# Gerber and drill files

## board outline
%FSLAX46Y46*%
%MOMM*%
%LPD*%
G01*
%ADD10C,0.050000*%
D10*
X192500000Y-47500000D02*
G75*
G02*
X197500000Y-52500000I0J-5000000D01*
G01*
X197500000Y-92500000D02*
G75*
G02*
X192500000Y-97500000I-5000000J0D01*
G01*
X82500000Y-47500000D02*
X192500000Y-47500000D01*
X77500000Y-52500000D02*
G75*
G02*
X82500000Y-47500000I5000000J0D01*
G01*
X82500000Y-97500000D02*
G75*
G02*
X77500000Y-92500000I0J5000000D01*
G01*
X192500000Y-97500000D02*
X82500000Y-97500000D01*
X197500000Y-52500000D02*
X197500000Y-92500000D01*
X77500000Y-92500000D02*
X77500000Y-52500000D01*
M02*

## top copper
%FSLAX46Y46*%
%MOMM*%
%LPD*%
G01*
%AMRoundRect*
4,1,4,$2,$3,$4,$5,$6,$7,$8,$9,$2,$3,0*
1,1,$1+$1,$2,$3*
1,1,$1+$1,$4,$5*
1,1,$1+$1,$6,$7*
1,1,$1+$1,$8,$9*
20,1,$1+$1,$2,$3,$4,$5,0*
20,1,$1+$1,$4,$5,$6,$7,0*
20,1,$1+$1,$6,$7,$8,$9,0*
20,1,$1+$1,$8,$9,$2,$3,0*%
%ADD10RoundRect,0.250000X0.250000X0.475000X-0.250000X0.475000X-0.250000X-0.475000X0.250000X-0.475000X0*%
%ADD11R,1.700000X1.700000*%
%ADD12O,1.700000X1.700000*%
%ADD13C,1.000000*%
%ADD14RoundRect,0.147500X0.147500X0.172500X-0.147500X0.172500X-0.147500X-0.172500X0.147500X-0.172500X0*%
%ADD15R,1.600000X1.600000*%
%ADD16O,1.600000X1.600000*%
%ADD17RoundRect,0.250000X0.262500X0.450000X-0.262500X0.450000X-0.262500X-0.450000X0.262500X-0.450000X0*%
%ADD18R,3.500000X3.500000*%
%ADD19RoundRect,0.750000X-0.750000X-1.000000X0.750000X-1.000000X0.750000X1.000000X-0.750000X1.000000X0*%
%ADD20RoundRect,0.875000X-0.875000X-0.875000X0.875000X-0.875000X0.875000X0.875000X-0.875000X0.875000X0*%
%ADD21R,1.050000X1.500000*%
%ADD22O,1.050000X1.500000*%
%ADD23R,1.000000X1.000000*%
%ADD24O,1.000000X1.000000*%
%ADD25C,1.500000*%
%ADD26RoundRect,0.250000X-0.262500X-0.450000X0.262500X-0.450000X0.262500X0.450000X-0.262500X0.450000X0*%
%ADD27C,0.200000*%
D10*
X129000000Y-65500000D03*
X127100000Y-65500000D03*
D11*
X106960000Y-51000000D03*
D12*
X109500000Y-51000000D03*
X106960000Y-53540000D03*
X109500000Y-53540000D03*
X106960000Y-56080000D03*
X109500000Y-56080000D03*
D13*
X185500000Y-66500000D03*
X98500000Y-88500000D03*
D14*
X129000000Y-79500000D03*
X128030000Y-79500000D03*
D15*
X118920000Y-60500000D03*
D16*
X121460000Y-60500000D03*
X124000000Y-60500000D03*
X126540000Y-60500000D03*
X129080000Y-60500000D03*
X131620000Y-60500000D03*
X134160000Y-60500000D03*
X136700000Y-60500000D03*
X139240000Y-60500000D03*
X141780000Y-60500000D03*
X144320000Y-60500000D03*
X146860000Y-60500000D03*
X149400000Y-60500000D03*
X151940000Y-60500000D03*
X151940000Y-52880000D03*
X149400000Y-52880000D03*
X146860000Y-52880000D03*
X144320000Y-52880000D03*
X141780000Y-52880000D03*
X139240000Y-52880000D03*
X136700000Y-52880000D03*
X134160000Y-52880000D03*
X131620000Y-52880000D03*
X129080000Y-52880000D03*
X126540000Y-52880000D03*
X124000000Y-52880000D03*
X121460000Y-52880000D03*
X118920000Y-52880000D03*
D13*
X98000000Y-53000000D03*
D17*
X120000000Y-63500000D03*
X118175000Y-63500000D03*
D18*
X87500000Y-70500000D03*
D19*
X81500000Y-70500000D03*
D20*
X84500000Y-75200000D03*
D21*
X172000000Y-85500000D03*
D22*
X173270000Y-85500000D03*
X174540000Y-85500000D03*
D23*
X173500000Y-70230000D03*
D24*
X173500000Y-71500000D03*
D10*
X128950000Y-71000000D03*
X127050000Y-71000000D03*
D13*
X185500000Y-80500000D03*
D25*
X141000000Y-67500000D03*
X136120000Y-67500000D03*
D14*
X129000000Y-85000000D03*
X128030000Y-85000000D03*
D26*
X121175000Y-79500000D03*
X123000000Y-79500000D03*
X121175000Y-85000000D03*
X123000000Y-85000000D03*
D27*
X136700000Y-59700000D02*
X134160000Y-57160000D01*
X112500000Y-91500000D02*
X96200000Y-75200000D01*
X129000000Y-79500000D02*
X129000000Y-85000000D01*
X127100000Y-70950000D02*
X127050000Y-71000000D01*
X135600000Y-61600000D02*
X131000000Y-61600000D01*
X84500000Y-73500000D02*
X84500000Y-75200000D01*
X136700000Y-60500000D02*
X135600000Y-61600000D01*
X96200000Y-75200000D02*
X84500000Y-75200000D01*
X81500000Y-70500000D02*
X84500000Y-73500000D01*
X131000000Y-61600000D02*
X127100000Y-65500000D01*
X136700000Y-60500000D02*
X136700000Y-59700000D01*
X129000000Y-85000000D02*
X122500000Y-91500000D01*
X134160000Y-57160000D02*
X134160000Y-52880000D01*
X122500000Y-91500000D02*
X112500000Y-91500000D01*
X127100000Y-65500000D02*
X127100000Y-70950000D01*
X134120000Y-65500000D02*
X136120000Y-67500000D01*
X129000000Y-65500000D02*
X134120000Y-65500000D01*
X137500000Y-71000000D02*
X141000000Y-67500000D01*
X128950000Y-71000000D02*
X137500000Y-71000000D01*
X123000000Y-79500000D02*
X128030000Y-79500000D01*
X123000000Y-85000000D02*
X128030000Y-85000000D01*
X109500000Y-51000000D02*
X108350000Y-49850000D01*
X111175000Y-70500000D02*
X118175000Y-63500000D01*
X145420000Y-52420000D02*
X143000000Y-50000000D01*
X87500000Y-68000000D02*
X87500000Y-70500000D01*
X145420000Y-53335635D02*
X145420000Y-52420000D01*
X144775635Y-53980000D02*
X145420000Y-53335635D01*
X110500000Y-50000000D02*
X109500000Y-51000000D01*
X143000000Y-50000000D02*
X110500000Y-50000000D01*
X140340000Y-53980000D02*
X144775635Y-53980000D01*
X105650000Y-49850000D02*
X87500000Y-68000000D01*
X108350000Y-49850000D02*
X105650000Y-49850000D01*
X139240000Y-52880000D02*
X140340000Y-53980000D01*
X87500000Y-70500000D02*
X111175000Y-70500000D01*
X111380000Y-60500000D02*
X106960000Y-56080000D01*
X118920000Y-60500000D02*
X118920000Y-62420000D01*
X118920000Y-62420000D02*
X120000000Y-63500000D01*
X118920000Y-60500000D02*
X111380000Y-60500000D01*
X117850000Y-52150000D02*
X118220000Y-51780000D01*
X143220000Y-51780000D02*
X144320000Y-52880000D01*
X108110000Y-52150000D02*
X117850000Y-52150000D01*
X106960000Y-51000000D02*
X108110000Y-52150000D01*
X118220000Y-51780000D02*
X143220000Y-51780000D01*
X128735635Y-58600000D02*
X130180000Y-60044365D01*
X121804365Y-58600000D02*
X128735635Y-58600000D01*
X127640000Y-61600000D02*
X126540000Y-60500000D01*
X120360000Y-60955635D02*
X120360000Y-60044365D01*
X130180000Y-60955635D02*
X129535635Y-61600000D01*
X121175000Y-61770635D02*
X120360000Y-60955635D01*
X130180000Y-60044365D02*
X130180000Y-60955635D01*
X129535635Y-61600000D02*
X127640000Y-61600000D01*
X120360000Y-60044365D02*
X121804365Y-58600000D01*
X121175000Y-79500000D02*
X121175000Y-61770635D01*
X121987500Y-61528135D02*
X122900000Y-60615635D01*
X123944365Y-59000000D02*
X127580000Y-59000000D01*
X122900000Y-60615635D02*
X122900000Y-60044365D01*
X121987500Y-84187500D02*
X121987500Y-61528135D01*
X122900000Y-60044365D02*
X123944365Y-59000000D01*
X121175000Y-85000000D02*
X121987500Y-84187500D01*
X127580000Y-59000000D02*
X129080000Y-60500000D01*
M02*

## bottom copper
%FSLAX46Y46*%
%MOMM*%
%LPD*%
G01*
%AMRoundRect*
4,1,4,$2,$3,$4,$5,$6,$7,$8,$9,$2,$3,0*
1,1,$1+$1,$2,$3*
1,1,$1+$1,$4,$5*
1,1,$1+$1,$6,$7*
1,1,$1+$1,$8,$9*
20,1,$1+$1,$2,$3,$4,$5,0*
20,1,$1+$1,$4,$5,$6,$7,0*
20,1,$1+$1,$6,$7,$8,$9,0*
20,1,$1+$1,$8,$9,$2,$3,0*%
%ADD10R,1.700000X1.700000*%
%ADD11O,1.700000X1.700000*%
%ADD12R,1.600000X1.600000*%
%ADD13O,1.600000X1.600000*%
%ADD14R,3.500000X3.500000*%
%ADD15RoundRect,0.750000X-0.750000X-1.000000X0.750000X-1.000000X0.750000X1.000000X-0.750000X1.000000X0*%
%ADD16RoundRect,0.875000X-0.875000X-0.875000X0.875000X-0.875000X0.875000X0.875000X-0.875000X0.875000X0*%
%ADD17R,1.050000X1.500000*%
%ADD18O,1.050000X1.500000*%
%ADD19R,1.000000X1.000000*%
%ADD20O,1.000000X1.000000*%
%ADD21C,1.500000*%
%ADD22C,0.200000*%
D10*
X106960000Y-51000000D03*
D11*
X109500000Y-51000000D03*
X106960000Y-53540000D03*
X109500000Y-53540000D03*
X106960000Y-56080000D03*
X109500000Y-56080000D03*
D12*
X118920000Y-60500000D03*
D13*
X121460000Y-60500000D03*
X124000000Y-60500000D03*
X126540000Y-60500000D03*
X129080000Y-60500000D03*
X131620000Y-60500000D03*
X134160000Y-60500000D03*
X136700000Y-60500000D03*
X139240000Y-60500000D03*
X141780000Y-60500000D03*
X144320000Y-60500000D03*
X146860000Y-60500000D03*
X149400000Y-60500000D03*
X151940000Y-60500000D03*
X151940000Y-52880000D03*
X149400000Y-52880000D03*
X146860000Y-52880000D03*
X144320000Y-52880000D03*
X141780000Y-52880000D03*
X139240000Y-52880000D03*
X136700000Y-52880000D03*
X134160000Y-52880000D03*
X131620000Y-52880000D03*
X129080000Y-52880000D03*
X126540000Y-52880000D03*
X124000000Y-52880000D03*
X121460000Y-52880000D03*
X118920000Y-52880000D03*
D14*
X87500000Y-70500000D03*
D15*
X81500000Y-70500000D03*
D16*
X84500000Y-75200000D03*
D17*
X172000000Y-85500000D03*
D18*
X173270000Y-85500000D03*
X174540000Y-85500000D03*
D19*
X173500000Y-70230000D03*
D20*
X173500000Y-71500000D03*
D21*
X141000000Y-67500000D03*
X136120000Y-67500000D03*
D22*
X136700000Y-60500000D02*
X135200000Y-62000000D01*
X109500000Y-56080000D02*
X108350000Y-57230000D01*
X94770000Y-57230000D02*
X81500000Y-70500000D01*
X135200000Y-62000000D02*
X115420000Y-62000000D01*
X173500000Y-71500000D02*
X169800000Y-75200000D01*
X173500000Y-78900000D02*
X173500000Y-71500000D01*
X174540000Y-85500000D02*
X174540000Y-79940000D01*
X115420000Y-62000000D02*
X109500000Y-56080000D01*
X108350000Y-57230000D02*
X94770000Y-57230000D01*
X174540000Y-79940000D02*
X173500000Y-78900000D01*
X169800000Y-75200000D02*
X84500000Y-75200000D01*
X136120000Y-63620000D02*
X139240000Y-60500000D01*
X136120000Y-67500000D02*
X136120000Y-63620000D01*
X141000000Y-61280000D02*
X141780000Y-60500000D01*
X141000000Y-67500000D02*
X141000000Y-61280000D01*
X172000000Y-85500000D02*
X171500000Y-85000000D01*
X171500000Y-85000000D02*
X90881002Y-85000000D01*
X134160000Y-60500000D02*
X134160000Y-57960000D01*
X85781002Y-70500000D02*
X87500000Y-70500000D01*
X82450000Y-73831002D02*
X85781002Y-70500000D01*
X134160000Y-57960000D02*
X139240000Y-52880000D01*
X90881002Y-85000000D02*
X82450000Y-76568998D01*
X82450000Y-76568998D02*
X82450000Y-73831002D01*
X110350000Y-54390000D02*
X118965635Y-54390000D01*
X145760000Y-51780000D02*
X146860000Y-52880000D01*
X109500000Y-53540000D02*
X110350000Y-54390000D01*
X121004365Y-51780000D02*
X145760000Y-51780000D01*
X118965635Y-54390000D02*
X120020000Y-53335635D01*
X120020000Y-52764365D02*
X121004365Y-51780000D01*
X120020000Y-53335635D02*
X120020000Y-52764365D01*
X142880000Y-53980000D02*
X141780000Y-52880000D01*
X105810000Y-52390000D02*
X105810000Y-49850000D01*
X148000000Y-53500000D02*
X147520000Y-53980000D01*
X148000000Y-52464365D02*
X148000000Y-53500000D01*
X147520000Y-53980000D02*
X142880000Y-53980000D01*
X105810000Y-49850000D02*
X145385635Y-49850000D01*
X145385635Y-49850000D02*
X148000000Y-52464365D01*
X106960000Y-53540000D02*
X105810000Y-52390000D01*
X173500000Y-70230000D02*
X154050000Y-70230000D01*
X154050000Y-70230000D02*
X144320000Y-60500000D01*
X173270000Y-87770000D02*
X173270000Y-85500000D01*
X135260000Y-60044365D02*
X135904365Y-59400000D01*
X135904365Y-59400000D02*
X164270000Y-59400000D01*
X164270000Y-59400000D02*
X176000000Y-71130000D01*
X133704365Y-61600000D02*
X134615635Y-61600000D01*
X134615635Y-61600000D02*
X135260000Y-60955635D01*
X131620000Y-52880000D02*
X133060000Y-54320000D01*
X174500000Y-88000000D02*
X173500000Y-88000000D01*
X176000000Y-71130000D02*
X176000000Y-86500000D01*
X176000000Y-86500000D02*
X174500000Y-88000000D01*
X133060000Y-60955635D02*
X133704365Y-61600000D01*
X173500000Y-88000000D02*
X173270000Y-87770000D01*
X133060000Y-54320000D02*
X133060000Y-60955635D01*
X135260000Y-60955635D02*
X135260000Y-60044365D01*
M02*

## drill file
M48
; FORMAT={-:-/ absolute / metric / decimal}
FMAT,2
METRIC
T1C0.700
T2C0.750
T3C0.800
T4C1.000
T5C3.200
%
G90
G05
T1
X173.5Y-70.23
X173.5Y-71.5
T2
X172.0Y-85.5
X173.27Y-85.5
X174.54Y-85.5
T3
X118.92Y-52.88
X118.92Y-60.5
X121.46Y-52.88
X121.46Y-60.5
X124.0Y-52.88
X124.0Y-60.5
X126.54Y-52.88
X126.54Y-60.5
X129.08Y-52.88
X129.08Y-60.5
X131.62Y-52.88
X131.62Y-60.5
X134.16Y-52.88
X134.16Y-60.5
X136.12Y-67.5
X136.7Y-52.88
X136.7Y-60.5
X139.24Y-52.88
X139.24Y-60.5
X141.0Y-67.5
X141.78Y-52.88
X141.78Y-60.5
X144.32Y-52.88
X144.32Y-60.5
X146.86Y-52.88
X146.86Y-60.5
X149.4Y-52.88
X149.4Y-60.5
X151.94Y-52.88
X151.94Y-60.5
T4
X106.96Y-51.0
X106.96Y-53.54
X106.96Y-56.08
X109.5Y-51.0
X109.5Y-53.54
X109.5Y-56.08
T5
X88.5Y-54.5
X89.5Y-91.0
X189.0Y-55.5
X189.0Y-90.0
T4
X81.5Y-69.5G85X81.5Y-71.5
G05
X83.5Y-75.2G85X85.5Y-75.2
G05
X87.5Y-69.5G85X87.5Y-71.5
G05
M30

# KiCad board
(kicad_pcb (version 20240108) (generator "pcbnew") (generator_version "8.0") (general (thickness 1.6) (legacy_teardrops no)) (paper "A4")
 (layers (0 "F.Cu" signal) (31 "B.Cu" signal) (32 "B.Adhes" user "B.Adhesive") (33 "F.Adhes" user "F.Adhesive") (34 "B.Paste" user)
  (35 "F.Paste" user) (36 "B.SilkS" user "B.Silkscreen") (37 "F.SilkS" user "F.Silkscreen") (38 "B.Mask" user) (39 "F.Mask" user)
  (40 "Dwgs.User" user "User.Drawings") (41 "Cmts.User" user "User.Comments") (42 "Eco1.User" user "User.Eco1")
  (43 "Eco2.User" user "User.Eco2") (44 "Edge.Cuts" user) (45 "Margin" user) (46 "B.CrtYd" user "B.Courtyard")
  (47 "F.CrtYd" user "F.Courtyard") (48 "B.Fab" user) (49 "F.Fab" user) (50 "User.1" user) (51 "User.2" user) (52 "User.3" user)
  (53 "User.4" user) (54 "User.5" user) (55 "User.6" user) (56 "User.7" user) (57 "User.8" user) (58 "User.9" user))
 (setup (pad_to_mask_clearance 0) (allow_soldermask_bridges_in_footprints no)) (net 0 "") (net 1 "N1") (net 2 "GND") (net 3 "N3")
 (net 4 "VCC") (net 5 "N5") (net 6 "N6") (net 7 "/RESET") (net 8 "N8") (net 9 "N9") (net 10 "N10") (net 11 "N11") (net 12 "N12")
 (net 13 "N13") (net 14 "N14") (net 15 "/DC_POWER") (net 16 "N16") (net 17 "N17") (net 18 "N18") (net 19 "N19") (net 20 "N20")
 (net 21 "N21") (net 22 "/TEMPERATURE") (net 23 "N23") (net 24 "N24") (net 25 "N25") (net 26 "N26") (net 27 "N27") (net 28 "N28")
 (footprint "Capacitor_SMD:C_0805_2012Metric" (layer "F.Cu") (at 128.05 65.5 180)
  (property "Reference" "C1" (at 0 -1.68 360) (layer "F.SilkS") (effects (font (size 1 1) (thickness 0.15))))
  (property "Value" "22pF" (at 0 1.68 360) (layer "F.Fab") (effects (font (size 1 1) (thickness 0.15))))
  (pad "1" smd roundrect (at -0.95 0 180) (size 1 1.45) (layers "F.Cu" "F.Paste" "F.Mask") (roundrect_rratio 0.25) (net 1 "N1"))
  (pad "2" smd roundrect (at 0.95 0 180) (size 1 1.45) (layers "F.Cu" "F.Paste" "F.Mask") (roundrect_rratio 0.25) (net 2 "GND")))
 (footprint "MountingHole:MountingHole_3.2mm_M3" (layer "F.Cu") (at 189 55.5)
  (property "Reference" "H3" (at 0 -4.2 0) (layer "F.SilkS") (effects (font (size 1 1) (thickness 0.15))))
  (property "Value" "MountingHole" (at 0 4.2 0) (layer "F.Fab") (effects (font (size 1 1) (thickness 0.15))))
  (pad "" np_thru_hole circle (at 0 0) (size 3.2 3.2) (drill 3.2) (layers "*.Cu" "*.Mask")))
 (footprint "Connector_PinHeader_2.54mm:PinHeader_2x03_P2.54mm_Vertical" (layer "F.Cu") (at 106.96 51)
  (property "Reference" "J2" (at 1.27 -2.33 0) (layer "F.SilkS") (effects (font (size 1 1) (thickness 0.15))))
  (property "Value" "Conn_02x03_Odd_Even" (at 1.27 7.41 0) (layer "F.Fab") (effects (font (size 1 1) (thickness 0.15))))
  (pad "1" thru_hole rect (at 0 0) (size 1.7 1.7) (drill 1) (layers "*.Cu" "*.Mask") (remove_unused_layers no) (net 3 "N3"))
  (pad "2" thru_hole oval (at 2.54 0) (size 1.7 1.7) (drill 1) (layers "*.Cu" "*.Mask") (remove_unused_layers no) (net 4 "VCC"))
  (pad "3" thru_hole oval (at 0 2.54) (size 1.7 1.7) (drill 1) (layers "*.Cu" "*.Mask") (remove_unused_layers no) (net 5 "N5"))
  (pad "4" thru_hole oval (at 2.54 2.54) (size 1.7 1.7) (drill 1) (layers "*.Cu" "*.Mask") (remove_unused_layers no) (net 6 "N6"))
  (pad "5" thru_hole oval (at 0 5.08) (size 1.7 1.7) (drill 1) (layers "*.Cu" "*.Mask") (remove_unused_layers no) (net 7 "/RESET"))
  (pad "6" thru_hole oval (at 2.54 5.08) (size 1.7 1.7) (drill 1) (layers "*.Cu" "*.Mask") (remove_unused_layers no) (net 2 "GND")))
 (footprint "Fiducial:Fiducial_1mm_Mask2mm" (layer "F.Cu") (at 185.5 66.5)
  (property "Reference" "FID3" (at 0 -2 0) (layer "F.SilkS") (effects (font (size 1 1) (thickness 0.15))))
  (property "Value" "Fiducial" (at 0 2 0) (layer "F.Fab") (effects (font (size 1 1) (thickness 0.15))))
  (pad "" smd circle (at 0 0) (size 1 1) (layers "F.Cu" "F.Mask") (solder_mask_margin 0.5) (clearance 0.5)))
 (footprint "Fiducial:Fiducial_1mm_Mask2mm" (layer "F.Cu") (at 98.5 88.5)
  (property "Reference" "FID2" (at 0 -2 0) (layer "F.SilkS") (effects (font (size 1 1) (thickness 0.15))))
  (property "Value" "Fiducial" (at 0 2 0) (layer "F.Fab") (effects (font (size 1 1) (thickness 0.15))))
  (pad "" smd circle (at 0 0) (size 1 1) (layers "F.Cu" "F.Mask") (solder_mask_margin 0.5) (clearance 0.5)))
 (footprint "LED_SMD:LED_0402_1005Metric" (layer "F.Cu") (at 128.515 79.5 180)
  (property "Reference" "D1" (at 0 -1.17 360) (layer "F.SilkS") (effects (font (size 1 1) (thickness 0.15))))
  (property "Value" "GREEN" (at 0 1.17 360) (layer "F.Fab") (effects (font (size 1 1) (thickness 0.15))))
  (pad "1" smd roundrect (at -0.485 0 180) (size 0.59 0.64) (layers "F.Cu" "F.Paste" "F.Mask") (roundrect_rratio 0.25) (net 2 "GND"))
  (pad "2" smd roundrect (at 0.485 0 180) (size 0.59 0.64) (layers "F.Cu" "F.Paste" "F.Mask") (roundrect_rratio 0.25) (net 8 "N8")))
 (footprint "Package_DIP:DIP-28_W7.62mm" (layer "F.Cu") (at 118.92 60.5 90)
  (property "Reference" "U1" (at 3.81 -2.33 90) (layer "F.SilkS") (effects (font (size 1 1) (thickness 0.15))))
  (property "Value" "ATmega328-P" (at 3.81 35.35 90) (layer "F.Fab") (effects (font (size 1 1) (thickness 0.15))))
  (pad "1" thru_hole rect (at 0 0 90) (size 1.6 1.6) (drill 0.8) (layers "*.Cu" "*.Mask") (remove_unused_layers no) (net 7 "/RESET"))
  (pad "2" thru_hole oval (at 0 2.54 90) (size 1.6 1.6) (drill 0.8) (layers "*.Cu" "*.Mask") (remove_unused_layers no) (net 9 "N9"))
  (pad "3" thru_hole oval (at 0 5.08 90) (size 1.6 1.6) (drill 0.8) (layers "*.Cu" "*.Mask") (remove_unused_layers no) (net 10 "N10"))
  (pad "4" thru_hole oval (at 0 7.62 90) (size 1.6 1.6) (drill 0.8) (layers "*.Cu" "*.Mask") (remove_unused_layers no) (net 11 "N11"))
  (pad "5" thru_hole oval (at 0 10.16 90) (size 1.6 1.6) (drill 0.8) (layers "*.Cu" "*.Mask") (remove_unused_layers no) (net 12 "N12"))
  (pad "6" thru_hole oval (at 0 12.7 90) (size 1.6 1.6) (drill 0.8) (layers "*.Cu" "*.Mask") (remove_unused_layers no) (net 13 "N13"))
  (pad "7" thru_hole oval (at 0 15.24 90) (size 1.6 1.6) (drill 0.8) (layers "*.Cu" "*.Mask") (remove_unused_layers no) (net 4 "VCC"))
  (pad "8" thru_hole oval (at 0 17.78 90) (size 1.6 1.6) (drill 0.8) (layers "*.Cu" "*.Mask") (remove_unused_layers no) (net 2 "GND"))
  (pad "9" thru_hole oval (at 0 20.32 90) (size 1.6 1.6) (drill 0.8) (layers "*.Cu" "*.Mask") (remove_unused_layers no) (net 1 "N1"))
  (pad "10" thru_hole oval (at 0 22.86 90) (size 1.6 1.6) (drill 0.8) (layers "*.Cu" "*.Mask") (remove_unused_layers no) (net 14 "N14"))
  (pad "11" thru_hole oval (at 0 25.4 90) (size 1.6 1.6) (drill 0.8) (layers "*.Cu" "*.Mask") (remove_unused_layers no) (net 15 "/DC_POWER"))
  (pad "12" thru_hole oval (at 0 27.94 90) (size 1.6 1.6) (drill 0.8) (layers "*.Cu" "*.Mask") (remove_unused_layers no) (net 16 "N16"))
  (pad "13" thru_hole oval (at 0 30.48 90) (size 1.6 1.6) (drill 0.8) (layers "*.Cu" "*.Mask") (remove_unused_layers no) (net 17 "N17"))
  (pad "14" thru_hole oval (at 0 33.02 90) (size 1.6 1.6) (drill 0.8) (layers "*.Cu" "*.Mask") (remove_unused_layers no) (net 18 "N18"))
  (pad "15" thru_hole oval (at 7.62 33.02 90) (size 1.6 1.6) (drill 0.8) (layers "*.Cu" "*.Mask") (remove_unused_layers no) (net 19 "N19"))
  (pad "16" thru_hole oval (at 7.62 30.48 90) (size 1.6 1.6) (drill 0.8) (layers "*.Cu" "*.Mask") (remove_unused_layers no) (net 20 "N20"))
  (pad "17" thru_hole oval (at 7.62 27.94 90) (size 1.6 1.6) (drill 0.8) (layers "*.Cu" "*.Mask") (remove_unused_layers no) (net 6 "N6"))
  (pad "18" thru_hole oval (at 7.62 25.4 90) (size 1.6 1.6) (drill 0.8) (layers "*.Cu" "*.Mask") (remove_unused_layers no) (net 3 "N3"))
  (pad "19" thru_hole oval (at 7.62 22.86 90) (size 1.6 1.6) (drill 0.8) (layers "*.Cu" "*.Mask") (remove_unused_layers no) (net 5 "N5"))
  (pad "20" thru_hole oval (at 7.62 20.32 90) (size 1.6 1.6) (drill 0.8) (layers "*.Cu" "*.Mask") (remove_unused_layers no) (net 4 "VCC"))
  (pad "21" thru_hole oval (at 7.62 17.78 90) (size 1.6 1.6) (drill 0.8) (layers "*.Cu" "*.Mask") (remove_unused_layers no) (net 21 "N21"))
  (pad "22" thru_hole oval (at 7.62 15.24 90) (size 1.6 1.6) (drill 0.8) (layers "*.Cu" "*.Mask") (remove_unused_layers no) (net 2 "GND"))
  (pad "23" thru_hole oval (at 7.62 12.7 90) (size 1.6 1.6) (drill 0.8) (layers "*.Cu" "*.Mask") (remove_unused_layers no)
   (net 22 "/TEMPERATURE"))
  (pad "24" thru_hole oval (at 7.62 10.16 90) (size 1.6 1.6) (drill 0.8) (layers "*.Cu" "*.Mask") (remove_unused_layers no) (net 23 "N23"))
  (pad "25" thru_hole oval (at 7.62 7.62 90) (size 1.6 1.6) (drill 0.8) (layers "*.Cu" "*.Mask") (remove_unused_layers no) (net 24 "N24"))
  (pad "26" thru_hole oval (at 7.62 5.08 90) (size 1.6 1.6) (drill 0.8) (layers "*.Cu" "*.Mask") (remove_unused_layers no) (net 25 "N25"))
  (pad "27" thru_hole oval (at 7.62 2.54 90) (size 1.6 1.6) (drill 0.8) (layers "*.Cu" "*.Mask") (remove_unused_layers no) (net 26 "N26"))
  (pad "28" thru_hole oval (at 7.62 0 90) (size 1.6 1.6) (drill 0.8) (layers "*.Cu" "*.Mask") (remove_unused_layers no) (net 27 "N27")))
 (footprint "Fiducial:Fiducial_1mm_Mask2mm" (layer "F.Cu") (at 98 53)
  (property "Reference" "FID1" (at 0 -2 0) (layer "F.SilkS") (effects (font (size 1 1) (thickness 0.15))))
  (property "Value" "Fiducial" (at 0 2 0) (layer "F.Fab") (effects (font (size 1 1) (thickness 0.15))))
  (pad "" smd circle (at 0 0) (size 1 1) (layers "F.Cu" "F.Mask") (solder_mask_margin 0.5) (clearance 0.5)))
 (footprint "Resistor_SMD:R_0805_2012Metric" (layer "F.Cu") (at 119.0875 63.5 180)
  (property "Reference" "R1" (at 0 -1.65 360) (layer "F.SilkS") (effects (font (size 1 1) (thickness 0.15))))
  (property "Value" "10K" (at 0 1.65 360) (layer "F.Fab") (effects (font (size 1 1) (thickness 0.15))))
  (pad "1" smd roundrect (at -0.9125 0 180) (size 1.025 1.4) (layers "F.Cu" "F.Paste" "F.Mask") (roundrect_rratio 0.243902) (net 7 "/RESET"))
  (pad "2" smd roundrect (at 0.9125 0 180) (size 1.025 1.4) (layers "F.Cu" "F.Paste" "F.Mask") (roundrect_rratio 0.243902) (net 4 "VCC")))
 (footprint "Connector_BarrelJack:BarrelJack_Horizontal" (layer "F.Cu") (at 87.5 70.5)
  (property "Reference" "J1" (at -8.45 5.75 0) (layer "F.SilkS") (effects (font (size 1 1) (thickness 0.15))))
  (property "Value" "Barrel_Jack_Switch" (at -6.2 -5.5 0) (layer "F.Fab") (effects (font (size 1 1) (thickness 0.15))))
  (pad "1" thru_hole rect (at 0 0) (size 3.5 3.5) (drill oval 1 3) (layers "*.Cu" "*.Mask") (remove_unused_layers no) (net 4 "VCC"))
  (pad "2" thru_hole roundrect (at -6 0) (size 3 3.5) (drill oval 1 3) (layers "*.Cu" "*.Mask") (remove_unused_layers no)
   (roundrect_rratio 0.25) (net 2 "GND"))
  (pad "3" thru_hole roundrect (at -3 4.7) (size 3.5 3.5) (drill oval 3 1) (layers "*.Cu" "*.Mask") (remove_unused_layers no)
   (roundrect_rratio 0.25) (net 2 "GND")))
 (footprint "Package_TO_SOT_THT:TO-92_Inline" (layer "F.Cu") (at 172 85.5)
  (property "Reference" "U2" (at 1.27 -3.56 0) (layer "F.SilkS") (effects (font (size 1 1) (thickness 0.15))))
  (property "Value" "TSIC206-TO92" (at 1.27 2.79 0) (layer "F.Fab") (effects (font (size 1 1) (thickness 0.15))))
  (pad "1" thru_hole rect (at 0 0) (size 1.05 1.5) (drill 0.75) (layers "*.Cu" "*.Mask") (remove_unused_layers no) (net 4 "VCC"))
  (pad "2" thru_hole oval (at 1.27 0) (size 1.05 1.5) (drill 0.75) (layers "*.Cu" "*.Mask") (remove_unused_layers no)
   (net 22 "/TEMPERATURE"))
  (pad "3" thru_hole oval (at 2.54 0) (size 1.05 1.5) (drill 0.75) (layers "*.Cu" "*.Mask") (remove_unused_layers no) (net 2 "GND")))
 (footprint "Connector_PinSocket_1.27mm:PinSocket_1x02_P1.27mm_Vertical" (layer "F.Cu") (at 173.5 70.23)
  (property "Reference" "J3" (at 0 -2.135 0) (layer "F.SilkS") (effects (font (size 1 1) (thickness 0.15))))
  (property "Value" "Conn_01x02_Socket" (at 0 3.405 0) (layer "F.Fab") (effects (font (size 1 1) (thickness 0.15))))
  (pad "1" thru_hole rect (at 0 0) (size 1 1) (drill 0.7) (layers "*.Cu" "*.Mask") (remove_unused_layers no) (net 15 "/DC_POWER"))
  (pad "2" thru_hole oval (at 0 1.27) (size 1 1) (drill 0.7) (layers "*.Cu" "*.Mask") (remove_unused_layers no) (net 2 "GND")))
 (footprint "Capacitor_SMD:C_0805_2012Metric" (layer "F.Cu") (at 128 71 180)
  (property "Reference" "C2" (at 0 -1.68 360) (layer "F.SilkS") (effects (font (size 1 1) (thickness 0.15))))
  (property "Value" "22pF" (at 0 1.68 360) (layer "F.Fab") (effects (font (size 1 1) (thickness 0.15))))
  (pad "1" smd roundrect (at -0.95 0 180) (size 1 1.45) (layers "F.Cu" "F.Paste" "F.Mask") (roundrect_rratio 0.25) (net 14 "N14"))
  (pad "2" smd roundrect (at 0.95 0 180) (size 1 1.45) (layers "F.Cu" "F.Paste" "F.Mask") (roundrect_rratio 0.25) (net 2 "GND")))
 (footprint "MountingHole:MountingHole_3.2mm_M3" (layer "F.Cu") (at 88.5 54.5)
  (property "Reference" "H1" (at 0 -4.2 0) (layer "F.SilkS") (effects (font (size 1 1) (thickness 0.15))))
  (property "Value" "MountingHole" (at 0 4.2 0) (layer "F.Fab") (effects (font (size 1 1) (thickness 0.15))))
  (pad "" np_thru_hole circle (at 0 0) (size 3.2 3.2) (drill 3.2) (layers "*.Cu" "*.Mask")))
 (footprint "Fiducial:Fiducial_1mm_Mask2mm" (layer "F.Cu") (at 185.5 80.5)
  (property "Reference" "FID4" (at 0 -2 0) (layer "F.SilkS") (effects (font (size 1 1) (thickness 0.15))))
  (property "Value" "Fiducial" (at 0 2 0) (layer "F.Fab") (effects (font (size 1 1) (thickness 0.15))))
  (pad "" smd circle (at 0 0) (size 1 1) (layers "F.Cu" "F.Mask") (solder_mask_margin 0.5) (clearance 0.5)))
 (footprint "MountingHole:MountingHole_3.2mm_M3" (layer "F.Cu") (at 89.5 91)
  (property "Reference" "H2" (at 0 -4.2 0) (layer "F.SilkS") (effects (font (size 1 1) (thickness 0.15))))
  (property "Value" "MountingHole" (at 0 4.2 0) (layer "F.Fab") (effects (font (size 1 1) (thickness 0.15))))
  (pad "" np_thru_hole circle (at 0 0) (size 3.2 3.2) (drill 3.2) (layers "*.Cu" "*.Mask")))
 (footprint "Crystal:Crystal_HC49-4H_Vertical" (layer "F.Cu") (at 141 67.5 180)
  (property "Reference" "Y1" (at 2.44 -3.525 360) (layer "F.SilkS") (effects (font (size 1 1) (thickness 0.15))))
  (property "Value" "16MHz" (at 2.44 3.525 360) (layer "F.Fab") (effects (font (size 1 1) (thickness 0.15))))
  (pad "1" thru_hole circle (at 0 0 180) (size 1.5 1.5) (drill 0.8) (layers "*.Cu" "*.Mask") (remove_unused_layers no) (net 14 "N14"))
  (pad "2" thru_hole circle (at 4.88 0 180) (size 1.5 1.5) (drill 0.8) (layers "*.Cu" "*.Mask") (remove_unused_layers no) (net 1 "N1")))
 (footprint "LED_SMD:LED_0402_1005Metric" (layer "F.Cu") (at 128.515 85 180)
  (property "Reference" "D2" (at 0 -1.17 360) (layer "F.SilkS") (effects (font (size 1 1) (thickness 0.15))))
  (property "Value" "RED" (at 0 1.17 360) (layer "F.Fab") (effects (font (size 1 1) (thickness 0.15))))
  (pad "1" smd roundrect (at -0.485 0 180) (size 0.59 0.64) (layers "F.Cu" "F.Paste" "F.Mask") (roundrect_rratio 0.25) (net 2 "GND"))
  (pad "2" smd roundrect (at 0.485 0 180) (size 0.59 0.64) (layers "F.Cu" "F.Paste" "F.Mask") (roundrect_rratio 0.25) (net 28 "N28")))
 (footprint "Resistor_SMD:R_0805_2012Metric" (layer "F.Cu") (at 122.0875 79.5)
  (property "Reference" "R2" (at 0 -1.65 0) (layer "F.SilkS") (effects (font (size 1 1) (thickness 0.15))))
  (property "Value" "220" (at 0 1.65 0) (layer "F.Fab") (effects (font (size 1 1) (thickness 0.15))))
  (pad "1" smd roundrect (at -0.9125 0) (size 1.025 1.4) (layers "F.Cu" "F.Paste" "F.Mask") (roundrect_rratio 0.243902) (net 11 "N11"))
  (pad "2" smd roundrect (at 0.9125 0) (size 1.025 1.4) (layers "F.Cu" "F.Paste" "F.Mask") (roundrect_rratio 0.243902) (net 8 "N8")))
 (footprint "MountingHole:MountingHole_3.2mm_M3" (layer "F.Cu") (at 189 90)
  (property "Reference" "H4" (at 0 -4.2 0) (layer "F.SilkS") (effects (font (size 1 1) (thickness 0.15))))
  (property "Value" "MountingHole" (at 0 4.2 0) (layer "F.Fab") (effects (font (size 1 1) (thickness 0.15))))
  (pad "" np_thru_hole circle (at 0 0) (size 3.2 3.2) (drill 3.2) (layers "*.Cu" "*.Mask")))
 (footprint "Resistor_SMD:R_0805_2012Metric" (layer "F.Cu") (at 122.0875 85)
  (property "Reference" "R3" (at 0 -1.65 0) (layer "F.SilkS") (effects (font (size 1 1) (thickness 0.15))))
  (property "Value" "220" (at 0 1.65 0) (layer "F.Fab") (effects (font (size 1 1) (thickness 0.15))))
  (pad "1" smd roundrect (at -0.9125 0) (size 1.025 1.4) (layers "F.Cu" "F.Paste" "F.Mask") (roundrect_rratio 0.243902) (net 12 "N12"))
  (pad "2" smd roundrect (at 0.9125 0) (size 1.025 1.4) (layers "F.Cu" "F.Paste" "F.Mask") (roundrect_rratio 0.243902) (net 28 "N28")))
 (gr_arc (start 192.5 47.5) (mid 196.035534 48.964466) (end 197.5 52.5) (stroke (width 0.05) (type default)) (layer "Edge.Cuts"))
 (gr_arc (start 197.5 92.5) (mid 196.035534 96.035534) (end 192.5 97.5) (stroke (width 0.05) (type default)) (layer "Edge.Cuts"))
 (gr_line (start 82.5 47.5) (end 192.5 47.5) (stroke (width 0.05) (type default)) (layer "Edge.Cuts"))
 (gr_arc (start 77.5 52.5) (mid 78.964466 48.964466) (end 82.5 47.5) (stroke (width 0.05) (type default)) (layer "Edge.Cuts"))
 (gr_arc (start 82.5 97.5) (mid 78.964466 96.035534) (end 77.5 92.5) (stroke (width 0.05) (type default)) (layer "Edge.Cuts"))
 (gr_line (start 192.5 97.5) (end 82.5 97.5) (stroke (width 0.05) (type default)) (layer "Edge.Cuts"))
 (gr_line (start 197.5 52.5) (end 197.5 92.5) (stroke (width 0.05) (type default)) (layer "Edge.Cuts"))
 (gr_line (start 77.5 92.5) (end 77.5 52.5) (stroke (width 0.05) (type default)) (layer "Edge.Cuts"))
 (segment (start 136.7 59.7) (end 134.16 57.16) (width 0.2) (layer "F.Cu") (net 2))
 (segment (start 112.5 91.5) (end 96.2 75.2) (width 0.2) (layer "F.Cu") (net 2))
 (segment (start 129 79.5) (end 129 85) (width 0.2) (layer "F.Cu") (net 2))
 (segment (start 127.1 70.95) (end 127.05 71) (width 0.2) (layer "F.Cu") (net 2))
 (segment (start 135.6 61.6) (end 131 61.6) (width 0.2) (layer "F.Cu") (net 2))
 (segment (start 84.5 73.5) (end 84.5 75.2) (width 0.2) (layer "F.Cu") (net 2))
 (segment (start 136.7 60.5) (end 135.6 61.6) (width 0.2) (layer "F.Cu") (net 2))
 (segment (start 96.2 75.2) (end 84.5 75.2) (width 0.2) (layer "F.Cu") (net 2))
 (segment (start 81.5 70.5) (end 84.5 73.5) (width 0.2) (layer "F.Cu") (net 2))
 (segment (start 131 61.6) (end 127.1 65.5) (width 0.2) (layer "F.Cu") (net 2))
 (segment (start 136.7 60.5) (end 136.7 59.7) (width 0.2) (layer "F.Cu") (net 2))
 (segment (start 129 85) (end 122.5 91.5) (width 0.2) (layer "F.Cu") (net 2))
 (segment (start 134.16 57.16) (end 134.16 52.88) (width 0.2) (layer "F.Cu") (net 2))
 (segment (start 122.5 91.5) (end 112.5 91.5) (width 0.2) (layer "F.Cu") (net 2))
 (segment (start 127.1 65.5) (end 127.1 70.95) (width 0.2) (layer "F.Cu") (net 2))
 (segment (start 136.7 60.5) (end 135.2 62) (width 0.2) (layer "B.Cu") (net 2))
 (segment (start 109.5 56.08) (end 108.35 57.23) (width 0.2) (layer "B.Cu") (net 2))
 (segment (start 94.77 57.23) (end 81.5 70.5) (width 0.2) (layer "B.Cu") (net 2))
 (segment (start 135.2 62) (end 115.42 62) (width 0.2) (layer "B.Cu") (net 2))
 (segment (start 173.5 71.5) (end 169.8 75.2) (width 0.2) (layer "B.Cu") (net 2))
 (segment (start 173.5 78.9) (end 173.5 71.5) (width 0.2) (layer "B.Cu") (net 2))
 (segment (start 174.54 85.5) (end 174.54 79.94) (width 0.2) (layer "B.Cu") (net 2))
 (segment (start 115.42 62) (end 109.5 56.08) (width 0.2) (layer "B.Cu") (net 2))
 (segment (start 108.35 57.23) (end 94.77 57.23) (width 0.2) (layer "B.Cu") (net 2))
 (segment (start 174.54 79.94) (end 173.5 78.9) (width 0.2) (layer "B.Cu") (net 2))
 (segment (start 169.8 75.2) (end 84.5 75.2) (width 0.2) (layer "B.Cu") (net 2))
 (segment (start 134.12 65.5) (end 136.12 67.5) (width 0.2) (layer "F.Cu") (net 1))
 (segment (start 129 65.5) (end 134.12 65.5) (width 0.2) (layer "F.Cu") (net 1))
 (segment (start 136.12 63.62) (end 139.24 60.5) (width 0.2) (layer "B.Cu") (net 1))
 (segment (start 136.12 67.5) (end 136.12 63.62) (width 0.2) (layer "B.Cu") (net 1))
 (segment (start 137.5 71) (end 141 67.5) (width 0.2) (layer "F.Cu") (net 14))
 (segment (start 128.95 71) (end 137.5 71) (width 0.2) (layer "F.Cu") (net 14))
 (segment (start 141 61.28) (end 141.78 60.5) (width 0.2) (layer "B.Cu") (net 14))
 (segment (start 141 67.5) (end 141 61.28) (width 0.2) (layer "B.Cu") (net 14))
 (segment (start 123 79.5) (end 128.03 79.5) (width 0.2) (layer "F.Cu") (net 8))
 (segment (start 123 85) (end 128.03 85) (width 0.2) (layer "F.Cu") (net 28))
 (segment (start 109.5 51) (end 108.35 49.85) (width 0.2) (layer "F.Cu") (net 4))
 (segment (start 111.175 70.5) (end 118.175 63.5) (width 0.2) (layer "F.Cu") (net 4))
 (segment (start 145.42 52.42) (end 143 50) (width 0.2) (layer "F.Cu") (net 4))
 (segment (start 87.5 68) (end 87.5 70.5) (width 0.2) (layer "F.Cu") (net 4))
 (segment (start 145.42 53.335635) (end 145.42 52.42) (width 0.2) (layer "F.Cu") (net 4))
 (segment (start 144.775635 53.98) (end 145.42 53.335635) (width 0.2) (layer "F.Cu") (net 4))
 (segment (start 110.5 50) (end 109.5 51) (width 0.2) (layer "F.Cu") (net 4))
 (segment (start 143 50) (end 110.5 50) (width 0.2) (layer "F.Cu") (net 4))
 (segment (start 140.34 53.98) (end 144.775635 53.98) (width 0.2) (layer "F.Cu") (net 4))
 (segment (start 105.65 49.85) (end 87.5 68) (width 0.2) (layer "F.Cu") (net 4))
 (segment (start 108.35 49.85) (end 105.65 49.85) (width 0.2) (layer "F.Cu") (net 4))
 (segment (start 139.24 52.88) (end 140.34 53.98) (width 0.2) (layer "F.Cu") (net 4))
 (segment (start 87.5 70.5) (end 111.175 70.5) (width 0.2) (layer "F.Cu") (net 4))
 (segment (start 172 85.5) (end 171.5 85) (width 0.2) (layer "B.Cu") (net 4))
 (segment (start 171.5 85) (end 90.881002 85) (width 0.2) (layer "B.Cu") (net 4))
 (segment (start 134.16 60.5) (end 134.16 57.96) (width 0.2) (layer "B.Cu") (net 4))
 (segment (start 85.781002 70.5) (end 87.5 70.5) (width 0.2) (layer "B.Cu") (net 4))
 (segment (start 82.45 73.831002) (end 85.781002 70.5) (width 0.2) (layer "B.Cu") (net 4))
 (segment (start 134.16 57.96) (end 139.24 52.88) (width 0.2) (layer "B.Cu") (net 4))
 (segment (start 90.881002 85) (end 82.45 76.568998) (width 0.2) (layer "B.Cu") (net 4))
 (segment (start 82.45 76.568998) (end 82.45 73.831002) (width 0.2) (layer "B.Cu") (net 4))
 (segment (start 110.35 54.39) (end 118.965635 54.39) (width 0.2) (layer "B.Cu") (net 6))
 (segment (start 145.76 51.78) (end 146.86 52.88) (width 0.2) (layer "B.Cu") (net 6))
 (segment (start 109.5 53.54) (end 110.35 54.39) (width 0.2) (layer "B.Cu") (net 6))
 (segment (start 121.004365 51.78) (end 145.76 51.78) (width 0.2) (layer "B.Cu") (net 6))
 (segment (start 118.965635 54.39) (end 120.02 53.335635) (width 0.2) (layer "B.Cu") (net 6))
 (segment (start 120.02 52.764365) (end 121.004365 51.78) (width 0.2) (layer "B.Cu") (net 6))
 (segment (start 120.02 53.335635) (end 120.02 52.764365) (width 0.2) (layer "B.Cu") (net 6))
 (segment (start 111.38 60.5) (end 106.96 56.08) (width 0.2) (layer "F.Cu") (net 7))
 (segment (start 118.92 60.5) (end 118.92 62.42) (width 0.2) (layer "F.Cu") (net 7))
 (segment (start 118.92 62.42) (end 120 63.5) (width 0.2) (layer "F.Cu") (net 7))
 (segment (start 118.92 60.5) (end 111.38 60.5) (width 0.2) (layer "F.Cu") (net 7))
 (segment (start 142.88 53.98) (end 141.78 52.88) (width 0.2) (layer "B.Cu") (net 5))
 (segment (start 105.81 52.39) (end 105.81 49.85) (width 0.2) (layer "B.Cu") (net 5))
 (segment (start 148 53.5) (end 147.52 53.98) (width 0.2) (layer "B.Cu") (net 5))
 (segment (start 148 52.464365) (end 148 53.5) (width 0.2) (layer "B.Cu") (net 5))
 (segment (start 147.52 53.98) (end 142.88 53.98) (width 0.2) (layer "B.Cu") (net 5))
 (segment (start 105.81 49.85) (end 145.385635 49.85) (width 0.2) (layer "B.Cu") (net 5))
 (segment (start 145.385635 49.85) (end 148 52.464365) (width 0.2) (layer "B.Cu") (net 5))
 (segment (start 106.96 53.54) (end 105.81 52.39) (width 0.2) (layer "B.Cu") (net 5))
 (segment (start 117.85 52.15) (end 118.22 51.78) (width 0.2) (layer "F.Cu") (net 3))
 (segment (start 143.22 51.78) (end 144.32 52.88) (width 0.2) (layer "F.Cu") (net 3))
 (segment (start 108.11 52.15) (end 117.85 52.15) (width 0.2) (layer "F.Cu") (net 3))
 (segment (start 106.96 51) (end 108.11 52.15) (width 0.2) (layer "F.Cu") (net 3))
 (segment (start 118.22 51.78) (end 143.22 51.78) (width 0.2) (layer "F.Cu") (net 3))
 (segment (start 173.5 70.23) (end 154.05 70.23) (width 0.2) (layer "B.Cu") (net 15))
 (segment (start 154.05 70.23) (end 144.32 60.5) (width 0.2) (layer "B.Cu") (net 15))
 (segment (start 128.735635 58.6) (end 130.18 60.044365) (width 0.2) (layer "F.Cu") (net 11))
 (segment (start 121.804365 58.6) (end 128.735635 58.6) (width 0.2) (layer "F.Cu") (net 11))
 (segment (start 127.64 61.6) (end 126.54 60.5) (width 0.2) (layer "F.Cu") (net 11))
 (segment (start 120.36 60.955635) (end 120.36 60.044365) (width 0.2) (layer "F.Cu") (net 11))
 (segment (start 130.18 60.955635) (end 129.535635 61.6) (width 0.2) (layer "F.Cu") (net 11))
 (segment (start 121.175 61.770635) (end 120.36 60.955635) (width 0.2) (layer "F.Cu") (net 11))
 (segment (start 130.18 60.044365) (end 130.18 60.955635) (width 0.2) (layer "F.Cu") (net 11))
 (segment (start 129.535635 61.6) (end 127.64 61.6) (width 0.2) (layer "F.Cu") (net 11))
 (segment (start 120.36 60.044365) (end 121.804365 58.6) (width 0.2) (layer "F.Cu") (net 11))
 (segment (start 121.175 79.5) (end 121.175 61.770635) (width 0.2) (layer "F.Cu") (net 11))
 (segment (start 121.9875 61.528135) (end 122.9 60.615635) (width 0.2) (layer "F.Cu") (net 12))
 (segment (start 123.944365 59) (end 127.58 59) (width 0.2) (layer "F.Cu") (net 12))
 (segment (start 122.9 60.615635) (end 122.9 60.044365) (width 0.2) (layer "F.Cu") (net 12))
 (segment (start 121.9875 84.1875) (end 121.9875 61.528135) (width 0.2) (layer "F.Cu") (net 12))
 (segment (start 122.9 60.044365) (end 123.944365 59) (width 0.2) (layer "F.Cu") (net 12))
 (segment (start 121.175 85) (end 121.9875 84.1875) (width 0.2) (layer "F.Cu") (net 12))
 (segment (start 127.58 59) (end 129.08 60.5) (width 0.2) (layer "F.Cu") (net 12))
 (segment (start 173.27 87.77) (end 173.27 85.5) (width 0.2) (layer "B.Cu") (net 22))
 (segment (start 135.26 60.044365) (end 135.904365 59.4) (width 0.2) (layer "B.Cu") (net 22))
 (segment (start 135.904365 59.4) (end 164.27 59.4) (width 0.2) (layer "B.Cu") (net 22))
 (segment (start 164.27 59.4) (end 176 71.13) (width 0.2) (layer "B.Cu") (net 22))
 (segment (start 133.704365 61.6) (end 134.615635 61.6) (width 0.2) (layer "B.Cu") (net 22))
 (segment (start 134.615635 61.6) (end 135.26 60.955635) (width 0.2) (layer "B.Cu") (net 22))
 (segment (start 131.62 52.88) (end 133.06 54.32) (width 0.2) (layer "B.Cu") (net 22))
 (segment (start 174.5 88) (end 173.5 88) (width 0.2) (layer "B.Cu") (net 22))
 (segment (start 176 71.13) (end 176 86.5) (width 0.2) (layer "B.Cu") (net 22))
 (segment (start 176 86.5) (end 174.5 88) (width 0.2) (layer "B.Cu") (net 22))
 (segment (start 133.06 60.955635) (end 133.704365 61.6) (width 0.2) (layer "B.Cu") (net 22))
 (segment (start 173.5 88) (end 173.27 87.77) (width 0.2) (layer "B.Cu") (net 22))
 (segment (start 133.06 54.32) (end 133.06 60.955635) (width 0.2) (layer "B.Cu") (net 22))
 (segment (start 135.26 60.955635) (end 135.26 60.044365) (width 0.2) (layer "B.Cu") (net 22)))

